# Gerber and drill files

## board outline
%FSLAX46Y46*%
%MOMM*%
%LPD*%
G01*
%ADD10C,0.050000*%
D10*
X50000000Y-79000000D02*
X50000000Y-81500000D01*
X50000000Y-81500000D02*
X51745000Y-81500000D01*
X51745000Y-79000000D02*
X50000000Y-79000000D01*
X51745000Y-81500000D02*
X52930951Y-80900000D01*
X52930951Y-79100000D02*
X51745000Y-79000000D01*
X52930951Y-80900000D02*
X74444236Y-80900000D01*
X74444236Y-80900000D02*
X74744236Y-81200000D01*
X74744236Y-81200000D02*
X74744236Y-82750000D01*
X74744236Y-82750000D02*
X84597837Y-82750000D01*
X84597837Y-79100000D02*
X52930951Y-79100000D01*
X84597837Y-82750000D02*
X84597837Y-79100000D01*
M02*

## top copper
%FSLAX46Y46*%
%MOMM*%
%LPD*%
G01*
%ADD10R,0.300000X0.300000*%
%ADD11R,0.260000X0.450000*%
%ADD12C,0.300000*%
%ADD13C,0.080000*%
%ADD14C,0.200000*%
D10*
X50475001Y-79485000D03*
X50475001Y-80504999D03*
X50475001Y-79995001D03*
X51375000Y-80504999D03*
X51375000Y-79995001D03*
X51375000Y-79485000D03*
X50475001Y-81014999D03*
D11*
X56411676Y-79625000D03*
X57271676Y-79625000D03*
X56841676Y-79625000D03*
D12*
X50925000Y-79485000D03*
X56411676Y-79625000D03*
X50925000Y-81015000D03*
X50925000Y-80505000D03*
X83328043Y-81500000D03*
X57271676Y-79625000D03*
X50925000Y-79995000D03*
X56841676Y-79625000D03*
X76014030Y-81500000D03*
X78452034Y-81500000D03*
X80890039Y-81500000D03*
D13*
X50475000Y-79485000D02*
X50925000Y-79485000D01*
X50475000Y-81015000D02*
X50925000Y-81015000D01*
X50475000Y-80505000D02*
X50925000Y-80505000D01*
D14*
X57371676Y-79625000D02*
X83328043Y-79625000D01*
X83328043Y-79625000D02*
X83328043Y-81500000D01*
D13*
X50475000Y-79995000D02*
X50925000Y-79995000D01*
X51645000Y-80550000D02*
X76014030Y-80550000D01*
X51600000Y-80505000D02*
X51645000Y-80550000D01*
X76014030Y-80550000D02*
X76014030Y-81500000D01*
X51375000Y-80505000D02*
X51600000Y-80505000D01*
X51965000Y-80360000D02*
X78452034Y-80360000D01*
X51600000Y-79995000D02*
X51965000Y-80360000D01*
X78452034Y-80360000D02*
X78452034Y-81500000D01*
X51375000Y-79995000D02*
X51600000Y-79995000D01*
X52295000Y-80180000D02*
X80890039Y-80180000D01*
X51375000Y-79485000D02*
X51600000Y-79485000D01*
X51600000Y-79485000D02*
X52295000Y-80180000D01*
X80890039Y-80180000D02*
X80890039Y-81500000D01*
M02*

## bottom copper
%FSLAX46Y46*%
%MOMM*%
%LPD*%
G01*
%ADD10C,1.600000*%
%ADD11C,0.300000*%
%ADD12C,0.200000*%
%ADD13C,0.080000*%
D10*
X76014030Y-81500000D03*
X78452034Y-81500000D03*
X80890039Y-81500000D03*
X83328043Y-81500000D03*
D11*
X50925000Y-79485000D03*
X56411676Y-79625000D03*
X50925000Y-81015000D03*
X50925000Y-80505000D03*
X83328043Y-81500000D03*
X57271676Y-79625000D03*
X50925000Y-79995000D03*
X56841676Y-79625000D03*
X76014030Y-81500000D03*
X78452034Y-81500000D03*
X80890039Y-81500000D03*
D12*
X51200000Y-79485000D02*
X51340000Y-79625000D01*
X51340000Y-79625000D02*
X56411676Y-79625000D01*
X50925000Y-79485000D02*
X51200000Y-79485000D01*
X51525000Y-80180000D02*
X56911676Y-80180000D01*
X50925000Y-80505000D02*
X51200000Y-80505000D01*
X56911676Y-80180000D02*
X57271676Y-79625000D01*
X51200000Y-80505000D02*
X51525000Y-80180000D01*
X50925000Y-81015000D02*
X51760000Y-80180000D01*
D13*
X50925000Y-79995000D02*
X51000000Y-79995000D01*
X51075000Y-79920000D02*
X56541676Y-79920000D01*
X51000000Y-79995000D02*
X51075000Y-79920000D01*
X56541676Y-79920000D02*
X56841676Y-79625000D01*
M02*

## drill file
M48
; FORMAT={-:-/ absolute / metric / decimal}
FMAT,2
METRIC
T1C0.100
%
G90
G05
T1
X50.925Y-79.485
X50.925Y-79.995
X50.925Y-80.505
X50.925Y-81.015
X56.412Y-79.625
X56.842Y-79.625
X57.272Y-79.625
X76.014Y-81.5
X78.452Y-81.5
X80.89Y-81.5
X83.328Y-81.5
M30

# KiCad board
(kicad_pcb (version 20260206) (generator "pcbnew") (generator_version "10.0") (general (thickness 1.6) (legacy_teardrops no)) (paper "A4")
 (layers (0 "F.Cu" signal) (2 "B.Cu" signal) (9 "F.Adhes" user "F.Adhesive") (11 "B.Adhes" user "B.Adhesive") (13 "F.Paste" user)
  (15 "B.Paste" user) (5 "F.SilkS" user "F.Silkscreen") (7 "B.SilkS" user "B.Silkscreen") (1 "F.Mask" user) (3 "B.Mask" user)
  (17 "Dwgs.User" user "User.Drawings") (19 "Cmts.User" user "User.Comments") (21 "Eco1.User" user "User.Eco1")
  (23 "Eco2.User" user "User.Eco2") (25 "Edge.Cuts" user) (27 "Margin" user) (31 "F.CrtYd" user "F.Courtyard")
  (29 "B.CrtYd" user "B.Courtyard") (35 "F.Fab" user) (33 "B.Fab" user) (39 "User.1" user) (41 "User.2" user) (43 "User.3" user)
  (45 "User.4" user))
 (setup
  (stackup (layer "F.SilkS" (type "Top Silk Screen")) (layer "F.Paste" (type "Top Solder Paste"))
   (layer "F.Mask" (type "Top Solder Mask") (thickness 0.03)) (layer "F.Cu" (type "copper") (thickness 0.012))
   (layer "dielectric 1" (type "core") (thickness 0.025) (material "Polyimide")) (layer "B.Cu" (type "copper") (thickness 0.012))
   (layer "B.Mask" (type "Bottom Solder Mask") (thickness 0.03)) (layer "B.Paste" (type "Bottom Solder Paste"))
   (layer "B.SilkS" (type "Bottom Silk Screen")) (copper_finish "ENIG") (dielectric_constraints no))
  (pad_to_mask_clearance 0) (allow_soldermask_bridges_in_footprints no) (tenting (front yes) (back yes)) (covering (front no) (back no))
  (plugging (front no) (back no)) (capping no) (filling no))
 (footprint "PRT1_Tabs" (layer "F.Cu") (at 56.841676 79.625)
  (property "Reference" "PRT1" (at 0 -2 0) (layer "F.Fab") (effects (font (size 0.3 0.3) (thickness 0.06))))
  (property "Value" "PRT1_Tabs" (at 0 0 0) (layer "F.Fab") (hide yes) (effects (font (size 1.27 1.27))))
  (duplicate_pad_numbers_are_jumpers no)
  (pad "1" smd rect (at -0.43 0) (size 0.26 0.45) (layers "F.Cu" "F.Mask") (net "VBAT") (solder_mask_margin 0.05) (thermal_bridge_angle 45))
  (pad "2" smd rect (at 0.43 0) (size 0.26 0.45) (layers "F.Cu" "F.Mask") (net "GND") (solder_mask_margin 0.05) (thermal_bridge_angle 45))
  (pad "3" smd rect (at 0 0) (size 0.26 0.45) (layers "F.Cu" "F.Mask") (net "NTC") (solder_mask_margin 0.05) (thermal_bridge_angle 45)))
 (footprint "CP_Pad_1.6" (layer "F.Cu") (at 83.328043 81.5)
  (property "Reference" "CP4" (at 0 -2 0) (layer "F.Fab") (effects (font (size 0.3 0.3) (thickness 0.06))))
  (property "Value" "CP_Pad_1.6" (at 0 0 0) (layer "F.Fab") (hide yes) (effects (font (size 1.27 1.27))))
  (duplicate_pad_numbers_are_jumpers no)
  (pad "1" smd circle (at 0 0) (size 1.6 1.6) (layers "B.Cu" "B.Mask") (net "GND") (solder_mask_margin 0.1)))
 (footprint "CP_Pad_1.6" (layer "F.Cu") (at 78.452034 81.5)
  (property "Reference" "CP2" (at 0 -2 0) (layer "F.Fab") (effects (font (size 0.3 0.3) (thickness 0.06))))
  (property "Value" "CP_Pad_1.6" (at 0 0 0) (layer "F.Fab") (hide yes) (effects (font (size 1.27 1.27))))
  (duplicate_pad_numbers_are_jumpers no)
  (pad "1" smd circle (at 0 0) (size 1.6 1.6) (layers "B.Cu" "B.Mask") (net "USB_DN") (solder_mask_margin 0.1)))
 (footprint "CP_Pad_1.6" (layer "F.Cu") (at 80.890039 81.5)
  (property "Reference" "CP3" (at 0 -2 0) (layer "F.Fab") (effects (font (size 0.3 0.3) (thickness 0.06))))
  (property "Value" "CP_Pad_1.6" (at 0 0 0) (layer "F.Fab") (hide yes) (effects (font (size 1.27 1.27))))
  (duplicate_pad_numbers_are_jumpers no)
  (pad "1" smd circle (at 0 0) (size 1.6 1.6) (layers "B.Cu" "B.Mask") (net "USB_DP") (solder_mask_margin 0.1)))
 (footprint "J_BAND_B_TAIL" (layer "F.Cu") (at 50.9 80.25)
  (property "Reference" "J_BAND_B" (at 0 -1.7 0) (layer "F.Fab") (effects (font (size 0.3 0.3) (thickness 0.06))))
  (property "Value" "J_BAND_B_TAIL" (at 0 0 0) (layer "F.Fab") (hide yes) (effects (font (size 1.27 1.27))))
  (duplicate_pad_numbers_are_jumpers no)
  (pad "1" smd rect (at -0.424999 -0.765) (size 0.3 0.3) (layers "F.Cu" "F.Mask") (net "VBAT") (solder_mask_margin 0.05)
   (thermal_bridge_angle 45))
  (pad "2" smd rect (at -0.424999 0.254999) (size 0.3 0.3) (layers "F.Cu" "F.Mask") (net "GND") (solder_mask_margin 0.05)
   (thermal_bridge_angle 45))
  (pad "3" smd rect (at -0.424999 -0.254999) (size 0.3 0.3) (layers "F.Cu" "F.Mask") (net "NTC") (solder_mask_margin 0.05)
   (thermal_bridge_angle 45))
  (pad "4" smd rect (at 0.475 0.254999) (size 0.3 0.3) (layers "F.Cu" "F.Mask") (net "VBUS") (solder_mask_margin 0.05)
   (thermal_bridge_angle 45))
  (pad "5" smd rect (at 0.475 -0.254999) (size 0.3 0.3) (layers "F.Cu" "F.Mask") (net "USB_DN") (solder_mask_margin 0.05)
   (thermal_bridge_angle 45))
  (pad "6" smd rect (at 0.475 -0.765) (size 0.3 0.3) (layers "F.Cu" "F.Mask") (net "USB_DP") (solder_mask_margin 0.05)
   (thermal_bridge_angle 45))
  (pad "7" smd rect (at -0.424999 0.764999) (size 0.3 0.3) (layers "F.Cu" "F.Mask") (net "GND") (solder_mask_margin 0.05)
   (thermal_bridge_angle 45)))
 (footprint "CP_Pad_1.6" (layer "F.Cu") (at 76.01403 81.5)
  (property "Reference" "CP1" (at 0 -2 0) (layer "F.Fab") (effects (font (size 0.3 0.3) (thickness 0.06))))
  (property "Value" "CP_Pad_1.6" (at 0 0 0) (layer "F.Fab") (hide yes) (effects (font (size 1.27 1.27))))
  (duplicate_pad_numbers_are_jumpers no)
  (pad "1" smd circle (at 0 0) (size 1.6 1.6) (layers "B.Cu" "B.Mask") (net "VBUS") (solder_mask_margin 0.1)))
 (gr_line (start 50 79) (end 50 81.5) (stroke (width 0.05) (type default)) (layer "Edge.Cuts"))
 (gr_line (start 50 81.5) (end 51.745 81.5) (stroke (width 0.05) (type default)) (layer "Edge.Cuts"))
 (gr_line (start 51.745 79) (end 50 79) (stroke (width 0.05) (type default)) (layer "Edge.Cuts"))
 (gr_line (start 51.745 81.5) (end 52.930951 80.9) (stroke (width 0.05) (type default)) (layer "Edge.Cuts"))
 (gr_line (start 52.930951 79.1) (end 51.745 79) (stroke (width 0.05) (type default)) (layer "Edge.Cuts"))
 (gr_line (start 52.930951 80.9) (end 74.444236 80.9) (stroke (width 0.05) (type default)) (layer "Edge.Cuts"))
 (gr_line (start 74.444236 80.9) (end 74.744236 81.2) (stroke (width 0.05) (type default)) (layer "Edge.Cuts"))
 (gr_line (start 74.744236 81.2) (end 74.744236 82.75) (stroke (width 0.05) (type default)) (layer "Edge.Cuts"))
 (gr_line (start 74.744236 82.75) (end 84.597837 82.75) (stroke (width 0.05) (type default)) (layer "Edge.Cuts"))
 (gr_line (start 84.597837 79.1) (end 52.930951 79.1) (stroke (width 0.05) (type default)) (layer "Edge.Cuts"))
 (gr_line (start 84.597837 82.75) (end 84.597837 79.1) (stroke (width 0.05) (type default)) (layer "Edge.Cuts"))
 (segment (start 50.475 79.485) (end 50.925 79.485) (width 0.08) (layer "F.Cu") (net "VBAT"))
 (via (at 56.411676 79.625) (size 0.3) (drill 0.1) (layers "F.Cu" "B.Cu") (tenting (front yes) (back yes)) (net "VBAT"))
 (via (at 50.925 79.485) (size 0.3) (drill 0.1) (layers "F.Cu" "B.Cu") (tenting (front yes) (back yes)) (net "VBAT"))
 (segment (start 51.2 79.485) (end 51.34 79.625) (width 0.2) (layer "B.Cu") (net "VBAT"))
 (segment (start 51.34 79.625) (end 56.411676 79.625) (width 0.2) (layer "B.Cu") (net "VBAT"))
 (segment (start 50.925 79.485) (end 51.2 79.485) (width 0.2) (layer "B.Cu") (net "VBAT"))
 (segment (start 50.475 81.015) (end 50.925 81.015) (width 0.08) (layer "F.Cu") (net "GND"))
 (segment (start 50.475 80.505) (end 50.925 80.505) (width 0.08) (layer "F.Cu") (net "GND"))
 (segment (start 57.371676 79.625) (end 83.328043 79.625) (width 0.2) (layer "F.Cu") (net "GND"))
 (segment (start 83.328043 79.625) (end 83.328043 81.5) (width 0.2) (layer "F.Cu") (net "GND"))
 (via (at 83.328043 81.5) (size 0.3) (drill 0.1) (layers "F.Cu" "B.Cu") (tenting (front yes) (back yes)) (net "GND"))
 (via (at 57.271676 79.625) (size 0.3) (drill 0.1) (layers "F.Cu" "B.Cu") (tenting (front yes) (back yes)) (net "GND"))
 (via (at 50.925 81.015) (size 0.3) (drill 0.1) (layers "F.Cu" "B.Cu") (tenting (front yes) (back yes)) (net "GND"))
 (via (at 50.925 80.505) (size 0.3) (drill 0.1) (layers "F.Cu" "B.Cu") (tenting (front yes) (back yes)) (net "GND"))
 (segment (start 51.2 80.505) (end 51.525 80.18) (width 0.2) (layer "B.Cu") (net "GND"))
 (segment (start 51.525 80.18) (end 56.911676 80.18) (width 0.2) (layer "B.Cu") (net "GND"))
 (segment (start 50.925 81.015) (end 51.76 80.18) (width 0.2) (layer "B.Cu") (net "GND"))
 (segment (start 50.925 80.505) (end 51.2 80.505) (width 0.2) (layer "B.Cu") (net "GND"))
 (segment (start 56.911676 80.18) (end 57.271676 79.625) (width 0.2) (layer "B.Cu") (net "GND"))
 (segment (start 50.475 79.995) (end 50.925 79.995) (width 0.08) (layer "F.Cu") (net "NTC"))
 (via (at 50.925 79.995) (size 0.3) (drill 0.1) (layers "F.Cu" "B.Cu") (tenting (front yes) (back yes)) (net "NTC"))
 (via (at 56.841676 79.625) (size 0.3) (drill 0.1) (layers "F.Cu" "B.Cu") (tenting (front yes) (back yes)) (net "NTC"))
 (segment (start 56.541676 79.92) (end 56.841676 79.625) (width 0.08) (layer "B.Cu") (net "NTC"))
 (segment (start 51 79.995) (end 51.075 79.92) (width 0.08) (layer "B.Cu") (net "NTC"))
 (segment (start 50.925 79.995) (end 51 79.995) (width 0.08) (layer "B.Cu") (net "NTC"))
 (segment (start 51.075 79.92) (end 56.541676 79.92) (width 0.08) (layer "B.Cu") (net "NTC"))
 (segment (start 51.375 80.505) (end 51.6 80.505) (width 0.08) (layer "F.Cu") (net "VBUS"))
 (segment (start 76.01403 80.55) (end 76.01403 81.5) (width 0.08) (layer "F.Cu") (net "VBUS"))
 (segment (start 51.645 80.55) (end 76.01403 80.55) (width 0.08) (layer "F.Cu") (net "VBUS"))
 (segment (start 51.6 80.505) (end 51.645 80.55) (width 0.08) (layer "F.Cu") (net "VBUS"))
 (via (at 76.01403 81.5) (size 0.3) (drill 0.1) (layers "F.Cu" "B.Cu") (tenting (front yes) (back yes)) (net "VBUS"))
 (segment (start 78.452034 80.36) (end 78.452034 81.5) (width 0.08) (layer "F.Cu") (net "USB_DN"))
 (segment (start 51.375 79.995) (end 51.6 79.995) (width 0.08) (layer "F.Cu") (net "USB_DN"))
 (segment (start 51.6 79.995) (end 51.965 80.36) (width 0.08) (layer "F.Cu") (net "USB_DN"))
 (segment (start 51.965 80.36) (end 78.452034 80.36) (width 0.08) (layer "F.Cu") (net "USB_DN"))
 (via (at 78.452034 81.5) (size 0.3) (drill 0.1) (layers "F.Cu" "B.Cu") (tenting (front yes) (back yes)) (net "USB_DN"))
 (segment (start 51.6 79.485) (end 52.295 80.18) (width 0.08) (layer "F.Cu") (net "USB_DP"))
 (segment (start 52.295 80.18) (end 80.890039 80.18) (width 0.08) (layer "F.Cu") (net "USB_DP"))
 (segment (start 51.375 79.485) (end 51.6 79.485) (width 0.08) (layer "F.Cu") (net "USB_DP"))
 (segment (start 80.890039 80.18) (end 80.890039 81.5) (width 0.08) (layer "F.Cu") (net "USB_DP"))
 (via (at 80.890039 81.5) (size 0.3) (drill 0.1) (layers "F.Cu" "B.Cu") (tenting (front yes) (back yes)) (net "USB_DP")))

